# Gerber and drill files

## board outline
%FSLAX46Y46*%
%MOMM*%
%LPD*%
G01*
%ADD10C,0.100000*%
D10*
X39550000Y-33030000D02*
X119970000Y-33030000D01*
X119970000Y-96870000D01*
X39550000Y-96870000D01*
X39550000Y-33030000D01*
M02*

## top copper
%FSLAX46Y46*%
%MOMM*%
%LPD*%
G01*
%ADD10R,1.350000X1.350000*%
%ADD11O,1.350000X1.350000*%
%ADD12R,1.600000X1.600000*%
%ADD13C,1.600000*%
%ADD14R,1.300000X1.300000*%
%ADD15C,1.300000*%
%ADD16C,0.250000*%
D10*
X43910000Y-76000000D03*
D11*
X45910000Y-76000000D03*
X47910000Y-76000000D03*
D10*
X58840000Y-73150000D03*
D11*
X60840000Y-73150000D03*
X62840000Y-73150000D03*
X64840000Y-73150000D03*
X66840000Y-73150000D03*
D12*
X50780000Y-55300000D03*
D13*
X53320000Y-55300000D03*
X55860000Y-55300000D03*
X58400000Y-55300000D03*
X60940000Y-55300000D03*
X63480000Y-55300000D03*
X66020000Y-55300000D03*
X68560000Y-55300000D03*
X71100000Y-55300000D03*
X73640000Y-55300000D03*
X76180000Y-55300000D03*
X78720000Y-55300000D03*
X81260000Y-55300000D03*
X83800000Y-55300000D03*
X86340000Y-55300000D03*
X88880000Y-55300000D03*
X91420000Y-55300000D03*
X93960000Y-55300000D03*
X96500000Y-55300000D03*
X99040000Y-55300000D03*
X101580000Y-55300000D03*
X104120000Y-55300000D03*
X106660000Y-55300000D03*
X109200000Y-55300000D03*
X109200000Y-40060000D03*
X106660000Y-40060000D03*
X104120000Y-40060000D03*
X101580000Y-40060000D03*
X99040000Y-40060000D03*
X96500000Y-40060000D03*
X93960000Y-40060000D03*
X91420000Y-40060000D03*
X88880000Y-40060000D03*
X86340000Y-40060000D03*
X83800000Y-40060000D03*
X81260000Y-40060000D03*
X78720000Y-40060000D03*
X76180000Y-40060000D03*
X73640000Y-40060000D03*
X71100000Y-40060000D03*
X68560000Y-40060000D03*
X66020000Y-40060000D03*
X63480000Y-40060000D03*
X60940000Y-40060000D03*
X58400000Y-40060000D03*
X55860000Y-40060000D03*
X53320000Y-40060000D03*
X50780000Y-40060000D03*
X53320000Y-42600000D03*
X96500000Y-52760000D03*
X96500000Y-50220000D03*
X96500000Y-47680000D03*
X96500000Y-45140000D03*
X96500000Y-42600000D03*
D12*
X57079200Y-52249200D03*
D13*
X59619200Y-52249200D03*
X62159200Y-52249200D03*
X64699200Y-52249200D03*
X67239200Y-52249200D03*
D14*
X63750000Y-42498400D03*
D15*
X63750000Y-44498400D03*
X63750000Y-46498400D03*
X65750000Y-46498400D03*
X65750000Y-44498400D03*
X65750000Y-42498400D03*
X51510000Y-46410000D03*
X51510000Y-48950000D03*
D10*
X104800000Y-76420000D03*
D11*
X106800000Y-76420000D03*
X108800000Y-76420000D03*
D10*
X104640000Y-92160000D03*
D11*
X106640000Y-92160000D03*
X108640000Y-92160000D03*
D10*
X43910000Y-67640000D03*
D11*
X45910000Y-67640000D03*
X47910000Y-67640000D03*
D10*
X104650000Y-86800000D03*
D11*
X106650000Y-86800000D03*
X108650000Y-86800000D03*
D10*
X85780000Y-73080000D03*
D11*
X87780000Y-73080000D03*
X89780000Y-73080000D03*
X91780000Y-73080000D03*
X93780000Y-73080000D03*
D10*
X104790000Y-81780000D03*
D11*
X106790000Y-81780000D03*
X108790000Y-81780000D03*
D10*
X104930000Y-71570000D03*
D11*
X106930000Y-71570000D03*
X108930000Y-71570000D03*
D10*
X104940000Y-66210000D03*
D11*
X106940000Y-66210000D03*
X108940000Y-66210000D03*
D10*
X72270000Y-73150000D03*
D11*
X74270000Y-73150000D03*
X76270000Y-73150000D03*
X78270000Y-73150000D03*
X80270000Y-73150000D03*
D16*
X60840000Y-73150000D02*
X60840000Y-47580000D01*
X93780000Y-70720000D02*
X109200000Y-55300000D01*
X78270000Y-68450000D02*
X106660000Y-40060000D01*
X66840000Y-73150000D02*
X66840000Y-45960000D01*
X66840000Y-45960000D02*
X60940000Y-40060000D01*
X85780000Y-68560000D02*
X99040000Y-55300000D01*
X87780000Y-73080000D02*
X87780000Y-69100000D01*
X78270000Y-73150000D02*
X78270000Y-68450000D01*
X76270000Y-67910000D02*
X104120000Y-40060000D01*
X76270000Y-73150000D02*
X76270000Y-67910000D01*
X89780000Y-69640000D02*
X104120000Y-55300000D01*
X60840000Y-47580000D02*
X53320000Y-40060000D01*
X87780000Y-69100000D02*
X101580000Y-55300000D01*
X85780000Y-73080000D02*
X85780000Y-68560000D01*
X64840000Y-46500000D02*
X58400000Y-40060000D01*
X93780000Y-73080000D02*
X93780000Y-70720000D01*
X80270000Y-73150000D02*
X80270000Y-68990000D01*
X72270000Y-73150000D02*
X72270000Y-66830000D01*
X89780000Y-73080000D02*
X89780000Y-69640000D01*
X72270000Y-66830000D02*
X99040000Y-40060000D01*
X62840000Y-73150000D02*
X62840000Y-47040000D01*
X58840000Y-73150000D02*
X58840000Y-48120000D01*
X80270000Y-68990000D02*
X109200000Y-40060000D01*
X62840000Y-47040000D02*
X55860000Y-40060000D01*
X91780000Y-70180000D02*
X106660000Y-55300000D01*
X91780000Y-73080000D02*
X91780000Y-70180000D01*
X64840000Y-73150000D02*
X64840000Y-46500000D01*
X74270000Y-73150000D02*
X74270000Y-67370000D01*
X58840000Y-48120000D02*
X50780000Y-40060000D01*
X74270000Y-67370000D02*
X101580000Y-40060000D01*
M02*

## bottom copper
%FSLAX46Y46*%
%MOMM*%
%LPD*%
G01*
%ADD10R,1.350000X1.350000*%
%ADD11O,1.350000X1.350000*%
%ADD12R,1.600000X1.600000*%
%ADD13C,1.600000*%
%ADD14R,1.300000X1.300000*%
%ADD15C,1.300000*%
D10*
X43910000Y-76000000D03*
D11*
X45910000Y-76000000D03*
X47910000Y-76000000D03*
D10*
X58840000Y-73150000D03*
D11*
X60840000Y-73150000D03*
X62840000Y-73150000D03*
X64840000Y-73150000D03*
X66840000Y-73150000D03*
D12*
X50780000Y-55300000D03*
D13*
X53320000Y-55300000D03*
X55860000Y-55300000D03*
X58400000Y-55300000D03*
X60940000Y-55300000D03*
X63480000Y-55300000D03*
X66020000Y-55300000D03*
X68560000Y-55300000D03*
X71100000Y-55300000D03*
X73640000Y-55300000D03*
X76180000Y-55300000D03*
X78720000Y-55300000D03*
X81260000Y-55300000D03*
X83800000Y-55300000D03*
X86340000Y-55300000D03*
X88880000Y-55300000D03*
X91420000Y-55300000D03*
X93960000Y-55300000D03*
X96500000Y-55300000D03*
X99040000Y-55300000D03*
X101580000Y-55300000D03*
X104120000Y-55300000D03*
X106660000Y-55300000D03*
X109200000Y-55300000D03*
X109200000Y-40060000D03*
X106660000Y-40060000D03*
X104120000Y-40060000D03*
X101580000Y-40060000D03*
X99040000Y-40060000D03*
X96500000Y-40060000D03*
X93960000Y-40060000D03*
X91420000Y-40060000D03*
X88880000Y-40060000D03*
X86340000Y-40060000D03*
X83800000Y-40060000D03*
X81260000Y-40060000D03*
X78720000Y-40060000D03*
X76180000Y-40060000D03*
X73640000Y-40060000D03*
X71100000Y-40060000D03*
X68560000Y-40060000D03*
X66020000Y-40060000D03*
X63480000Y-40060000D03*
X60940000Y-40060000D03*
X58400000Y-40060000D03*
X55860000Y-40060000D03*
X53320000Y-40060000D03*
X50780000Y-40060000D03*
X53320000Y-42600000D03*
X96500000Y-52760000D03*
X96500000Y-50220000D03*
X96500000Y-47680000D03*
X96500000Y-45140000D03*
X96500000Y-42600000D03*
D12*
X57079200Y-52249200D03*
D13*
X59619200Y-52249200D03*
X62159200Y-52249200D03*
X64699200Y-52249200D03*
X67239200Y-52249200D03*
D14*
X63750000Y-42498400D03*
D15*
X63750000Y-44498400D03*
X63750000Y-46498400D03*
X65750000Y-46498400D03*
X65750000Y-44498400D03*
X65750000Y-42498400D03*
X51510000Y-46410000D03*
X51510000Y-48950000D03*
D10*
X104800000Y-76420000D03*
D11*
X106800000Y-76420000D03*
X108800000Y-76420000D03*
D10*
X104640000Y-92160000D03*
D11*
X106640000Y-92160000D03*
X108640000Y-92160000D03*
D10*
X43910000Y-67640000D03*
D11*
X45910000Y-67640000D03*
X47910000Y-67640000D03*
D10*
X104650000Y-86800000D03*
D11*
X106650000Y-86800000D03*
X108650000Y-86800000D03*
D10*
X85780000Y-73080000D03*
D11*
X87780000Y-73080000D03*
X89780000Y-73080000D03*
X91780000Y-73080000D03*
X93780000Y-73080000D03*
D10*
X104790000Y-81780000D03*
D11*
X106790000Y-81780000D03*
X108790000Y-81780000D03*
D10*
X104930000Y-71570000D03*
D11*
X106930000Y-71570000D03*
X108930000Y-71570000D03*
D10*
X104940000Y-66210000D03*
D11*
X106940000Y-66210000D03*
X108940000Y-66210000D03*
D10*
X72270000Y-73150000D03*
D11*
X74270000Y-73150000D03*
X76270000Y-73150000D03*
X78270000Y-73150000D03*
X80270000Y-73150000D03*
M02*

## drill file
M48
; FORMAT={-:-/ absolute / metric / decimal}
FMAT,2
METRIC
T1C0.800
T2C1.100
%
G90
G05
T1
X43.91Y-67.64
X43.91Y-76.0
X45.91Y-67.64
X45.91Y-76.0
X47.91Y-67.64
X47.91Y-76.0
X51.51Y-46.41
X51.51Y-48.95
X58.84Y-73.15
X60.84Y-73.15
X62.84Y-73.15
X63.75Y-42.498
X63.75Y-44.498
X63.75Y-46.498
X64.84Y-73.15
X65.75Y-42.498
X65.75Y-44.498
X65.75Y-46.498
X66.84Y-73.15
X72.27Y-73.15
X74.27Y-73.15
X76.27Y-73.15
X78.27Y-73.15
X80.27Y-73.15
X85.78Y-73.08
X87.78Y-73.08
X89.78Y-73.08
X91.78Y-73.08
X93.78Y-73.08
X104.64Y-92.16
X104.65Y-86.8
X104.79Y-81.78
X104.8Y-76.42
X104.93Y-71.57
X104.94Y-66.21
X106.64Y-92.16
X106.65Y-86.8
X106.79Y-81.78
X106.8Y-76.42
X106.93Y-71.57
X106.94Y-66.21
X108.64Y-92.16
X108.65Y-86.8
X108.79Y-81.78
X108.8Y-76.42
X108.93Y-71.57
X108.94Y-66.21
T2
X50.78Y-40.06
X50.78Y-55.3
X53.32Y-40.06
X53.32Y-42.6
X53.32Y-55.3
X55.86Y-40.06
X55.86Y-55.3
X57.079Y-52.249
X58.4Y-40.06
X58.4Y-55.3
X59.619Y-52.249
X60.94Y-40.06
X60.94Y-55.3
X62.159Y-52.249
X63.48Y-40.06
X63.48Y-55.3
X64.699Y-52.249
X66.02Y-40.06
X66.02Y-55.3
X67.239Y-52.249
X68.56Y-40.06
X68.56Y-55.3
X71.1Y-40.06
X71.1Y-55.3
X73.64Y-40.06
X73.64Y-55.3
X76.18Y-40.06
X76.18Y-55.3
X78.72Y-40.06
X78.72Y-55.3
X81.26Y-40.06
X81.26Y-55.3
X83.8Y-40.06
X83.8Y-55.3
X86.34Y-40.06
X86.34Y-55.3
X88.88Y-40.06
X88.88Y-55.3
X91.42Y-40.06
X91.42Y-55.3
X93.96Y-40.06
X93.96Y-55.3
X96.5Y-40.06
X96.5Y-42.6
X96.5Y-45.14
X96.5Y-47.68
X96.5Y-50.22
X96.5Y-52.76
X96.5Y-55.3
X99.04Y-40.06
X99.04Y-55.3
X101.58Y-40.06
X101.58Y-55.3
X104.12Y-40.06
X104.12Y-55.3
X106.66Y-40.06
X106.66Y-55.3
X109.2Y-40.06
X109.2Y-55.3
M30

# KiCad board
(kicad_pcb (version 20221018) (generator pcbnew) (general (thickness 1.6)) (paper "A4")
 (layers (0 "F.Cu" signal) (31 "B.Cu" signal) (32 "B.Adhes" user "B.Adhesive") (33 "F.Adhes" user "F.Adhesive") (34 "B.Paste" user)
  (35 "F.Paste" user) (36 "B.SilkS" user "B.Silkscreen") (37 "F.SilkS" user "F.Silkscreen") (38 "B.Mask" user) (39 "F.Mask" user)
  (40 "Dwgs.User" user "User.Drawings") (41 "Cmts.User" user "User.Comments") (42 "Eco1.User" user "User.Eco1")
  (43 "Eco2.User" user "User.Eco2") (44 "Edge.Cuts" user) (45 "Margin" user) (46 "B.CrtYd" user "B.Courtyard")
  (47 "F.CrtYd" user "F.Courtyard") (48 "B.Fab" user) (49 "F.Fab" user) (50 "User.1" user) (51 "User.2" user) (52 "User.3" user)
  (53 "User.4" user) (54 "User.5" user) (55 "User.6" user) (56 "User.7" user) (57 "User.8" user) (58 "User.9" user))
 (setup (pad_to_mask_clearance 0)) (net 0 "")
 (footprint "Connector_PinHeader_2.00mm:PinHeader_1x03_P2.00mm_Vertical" (layer "F.Cu") (at 43.91 76 90)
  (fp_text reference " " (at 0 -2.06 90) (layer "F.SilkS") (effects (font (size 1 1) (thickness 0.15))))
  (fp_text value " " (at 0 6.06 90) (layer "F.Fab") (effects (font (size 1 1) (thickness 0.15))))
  (pad "1" thru_hole rect (at 0 0 90) (size 1.35 1.35) (drill 0.8) (layers "*.Cu" "*.Mask"))
  (pad "2" thru_hole oval (at 0 2 90) (size 1.35 1.35) (drill 0.8) (layers "*.Cu" "*.Mask"))
  (pad "3" thru_hole oval (at 0 4 90) (size 1.35 1.35) (drill 0.8) (layers "*.Cu" "*.Mask")))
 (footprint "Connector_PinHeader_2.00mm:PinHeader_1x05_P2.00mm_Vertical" (layer "F.Cu") (at 58.84 73.15 90)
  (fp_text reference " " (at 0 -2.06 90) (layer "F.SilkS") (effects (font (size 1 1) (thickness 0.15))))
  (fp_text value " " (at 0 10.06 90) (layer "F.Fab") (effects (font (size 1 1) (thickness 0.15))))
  (pad "1" thru_hole rect (at 0 0 90) (size 1.35 1.35) (drill 0.8) (layers "*.Cu" "*.Mask"))
  (pad "2" thru_hole oval (at 0 2 90) (size 1.35 1.35) (drill 0.8) (layers "*.Cu" "*.Mask"))
  (pad "3" thru_hole oval (at 0 4 90) (size 1.35 1.35) (drill 0.8) (layers "*.Cu" "*.Mask"))
  (pad "4" thru_hole oval (at 0 6 90) (size 1.35 1.35) (drill 0.8) (layers "*.Cu" "*.Mask"))
  (pad "5" thru_hole oval (at 0 8 90) (size 1.35 1.35) (drill 0.8) (layers "*.Cu" "*.Mask")))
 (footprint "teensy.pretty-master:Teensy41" (layer "F.Cu") (at 79.99 47.68)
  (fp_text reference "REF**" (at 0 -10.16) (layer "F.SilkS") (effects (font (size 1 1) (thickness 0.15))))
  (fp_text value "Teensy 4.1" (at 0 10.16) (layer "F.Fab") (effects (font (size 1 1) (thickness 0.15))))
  (pad "1" thru_hole rect (at -29.21 7.62) (size 1.6 1.6) (drill 1.1) (layers "*.Cu" "*.Mask"))
  (pad "2" thru_hole circle (at -26.67 7.62) (size 1.6 1.6) (drill 1.1) (layers "*.Cu" "*.Mask"))
  (pad "3" thru_hole circle (at -24.13 7.62) (size 1.6 1.6) (drill 1.1) (layers "*.Cu" "*.Mask"))
  (pad "4" thru_hole circle (at -21.59 7.62) (size 1.6 1.6) (drill 1.1) (layers "*.Cu" "*.Mask"))
  (pad "5" thru_hole circle (at -19.05 7.62) (size 1.6 1.6) (drill 1.1) (layers "*.Cu" "*.Mask"))
  (pad "6" thru_hole circle (at -16.51 7.62) (size 1.6 1.6) (drill 1.1) (layers "*.Cu" "*.Mask"))
  (pad "7" thru_hole circle (at -13.97 7.62) (size 1.6 1.6) (drill 1.1) (layers "*.Cu" "*.Mask"))
  (pad "8" thru_hole circle (at -11.43 7.62) (size 1.6 1.6) (drill 1.1) (layers "*.Cu" "*.Mask"))
  (pad "9" thru_hole circle (at -8.89 7.62) (size 1.6 1.6) (drill 1.1) (layers "*.Cu" "*.Mask"))
  (pad "10" thru_hole circle (at -6.35 7.62) (size 1.6 1.6) (drill 1.1) (layers "*.Cu" "*.Mask"))
  (pad "11" thru_hole circle (at -3.81 7.62) (size 1.6 1.6) (drill 1.1) (layers "*.Cu" "*.Mask"))
  (pad "12" thru_hole circle (at -1.27 7.62) (size 1.6 1.6) (drill 1.1) (layers "*.Cu" "*.Mask"))
  (pad "13" thru_hole circle (at 1.27 7.62) (size 1.6 1.6) (drill 1.1) (layers "*.Cu" "*.Mask"))
  (pad "14" thru_hole circle (at 3.81 7.62) (size 1.6 1.6) (drill 1.1) (layers "*.Cu" "*.Mask"))
  (pad "15" thru_hole circle (at 6.35 7.62) (size 1.6 1.6) (drill 1.1) (layers "*.Cu" "*.Mask"))
  (pad "16" thru_hole circle (at 8.89 7.62) (size 1.6 1.6) (drill 1.1) (layers "*.Cu" "*.Mask"))
  (pad "17" thru_hole circle (at 11.43 7.62) (size 1.6 1.6) (drill 1.1) (layers "*.Cu" "*.Mask"))
  (pad "18" thru_hole circle (at 13.97 7.62) (size 1.6 1.6) (drill 1.1) (layers "*.Cu" "*.Mask"))
  (pad "19" thru_hole circle (at 16.51 7.62) (size 1.6 1.6) (drill 1.1) (layers "*.Cu" "*.Mask"))
  (pad "20" thru_hole circle (at 19.05 7.62) (size 1.6 1.6) (drill 1.1) (layers "*.Cu" "*.Mask"))
  (pad "21" thru_hole circle (at 21.59 7.62) (size 1.6 1.6) (drill 1.1) (layers "*.Cu" "*.Mask"))
  (pad "22" thru_hole circle (at 24.13 7.62) (size 1.6 1.6) (drill 1.1) (layers "*.Cu" "*.Mask"))
  (pad "23" thru_hole circle (at 26.67 7.62) (size 1.6 1.6) (drill 1.1) (layers "*.Cu" "*.Mask"))
  (pad "24" thru_hole circle (at 29.21 7.62) (size 1.6 1.6) (drill 1.1) (layers "*.Cu" "*.Mask"))
  (pad "25" thru_hole circle (at 29.21 -7.62) (size 1.6 1.6) (drill 1.1) (layers "*.Cu" "*.Mask"))
  (pad "26" thru_hole circle (at 26.67 -7.62) (size 1.6 1.6) (drill 1.1) (layers "*.Cu" "*.Mask"))
  (pad "27" thru_hole circle (at 24.13 -7.62) (size 1.6 1.6) (drill 1.1) (layers "*.Cu" "*.Mask"))
  (pad "28" thru_hole circle (at 21.59 -7.62) (size 1.6 1.6) (drill 1.1) (layers "*.Cu" "*.Mask"))
  (pad "29" thru_hole circle (at 19.05 -7.62) (size 1.6 1.6) (drill 1.1) (layers "*.Cu" "*.Mask"))
  (pad "30" thru_hole circle (at 16.51 -7.62) (size 1.6 1.6) (drill 1.1) (layers "*.Cu" "*.Mask"))
  (pad "31" thru_hole circle (at 13.97 -7.62) (size 1.6 1.6) (drill 1.1) (layers "*.Cu" "*.Mask"))
  (pad "32" thru_hole circle (at 11.43 -7.62) (size 1.6 1.6) (drill 1.1) (layers "*.Cu" "*.Mask"))
  (pad "33" thru_hole circle (at 8.89 -7.62) (size 1.6 1.6) (drill 1.1) (layers "*.Cu" "*.Mask"))
  (pad "34" thru_hole circle (at 6.35 -7.62) (size 1.6 1.6) (drill 1.1) (layers "*.Cu" "*.Mask"))
  (pad "35" thru_hole circle (at 3.81 -7.62) (size 1.6 1.6) (drill 1.1) (layers "*.Cu" "*.Mask"))
  (pad "36" thru_hole circle (at 1.27 -7.62) (size 1.6 1.6) (drill 1.1) (layers "*.Cu" "*.Mask"))
  (pad "37" thru_hole circle (at -1.27 -7.62) (size 1.6 1.6) (drill 1.1) (layers "*.Cu" "*.Mask"))
  (pad "38" thru_hole circle (at -3.81 -7.62) (size 1.6 1.6) (drill 1.1) (layers "*.Cu" "*.Mask"))
  (pad "39" thru_hole circle (at -6.35 -7.62) (size 1.6 1.6) (drill 1.1) (layers "*.Cu" "*.Mask"))
  (pad "40" thru_hole circle (at -8.89 -7.62) (size 1.6 1.6) (drill 1.1) (layers "*.Cu" "*.Mask"))
  (pad "41" thru_hole circle (at -11.43 -7.62) (size 1.6 1.6) (drill 1.1) (layers "*.Cu" "*.Mask"))
  (pad "42" thru_hole circle (at -13.97 -7.62) (size 1.6 1.6) (drill 1.1) (layers "*.Cu" "*.Mask"))
  (pad "43" thru_hole circle (at -16.51 -7.62) (size 1.6 1.6) (drill 1.1) (layers "*.Cu" "*.Mask"))
  (pad "44" thru_hole circle (at -19.05 -7.62) (size 1.6 1.6) (drill 1.1) (layers "*.Cu" "*.Mask"))
  (pad "45" thru_hole circle (at -21.59 -7.62) (size 1.6 1.6) (drill 1.1) (layers "*.Cu" "*.Mask"))
  (pad "46" thru_hole circle (at -24.13 -7.62) (size 1.6 1.6) (drill 1.1) (layers "*.Cu" "*.Mask"))
  (pad "47" thru_hole circle (at -26.67 -7.62) (size 1.6 1.6) (drill 1.1) (layers "*.Cu" "*.Mask"))
  (pad "48" thru_hole circle (at -29.21 -7.62) (size 1.6 1.6) (drill 1.1) (layers "*.Cu" "*.Mask"))
  (pad "49" thru_hole circle (at -26.67 -5.08) (size 1.6 1.6) (drill 1.1) (layers "*.Cu" "*.Mask"))
  (pad "50" thru_hole circle (at 16.51 5.08) (size 1.6 1.6) (drill 1.1) (layers "*.Cu" "*.Mask"))
  (pad "51" thru_hole circle (at 16.51 2.54) (size 1.6 1.6) (drill 1.1) (layers "*.Cu" "*.Mask"))
  (pad "52" thru_hole circle (at 16.51 0) (size 1.6 1.6) (drill 1.1) (layers "*.Cu" "*.Mask"))
  (pad "53" thru_hole circle (at 16.51 -2.54) (size 1.6 1.6) (drill 1.1) (layers "*.Cu" "*.Mask"))
  (pad "54" thru_hole circle (at 16.51 -5.08) (size 1.6 1.6) (drill 1.1) (layers "*.Cu" "*.Mask"))
  (pad "55" thru_hole rect (at -22.9108 4.5692) (size 1.6 1.6) (drill 1.1) (layers "*.Cu" "*.Mask"))
  (pad "56" thru_hole circle (at -20.3708 4.5692) (size 1.6 1.6) (drill 1.1) (layers "*.Cu" "*.Mask"))
  (pad "57" thru_hole circle (at -17.8308 4.5692) (size 1.6 1.6) (drill 1.1) (layers "*.Cu" "*.Mask"))
  (pad "58" thru_hole circle (at -15.2908 4.5692) (size 1.6 1.6) (drill 1.1) (layers "*.Cu" "*.Mask"))
  (pad "59" thru_hole circle (at -12.7508 4.5692) (size 1.6 1.6) (drill 1.1) (layers "*.Cu" "*.Mask"))
  (pad "60" thru_hole rect (at -16.24 -5.1816) (size 1.3 1.3) (drill 0.8) (layers "*.Cu" "*.Mask"))
  (pad "61" thru_hole circle (at -16.24 -3.1816) (size 1.3 1.3) (drill 0.8) (layers "*.Cu" "*.Mask"))
  (pad "62" thru_hole circle (at -16.24 -1.1816) (size 1.3 1.3) (drill 0.8) (layers "*.Cu" "*.Mask"))
  (pad "63" thru_hole circle (at -14.24 -1.1816) (size 1.3 1.3) (drill 0.8) (layers "*.Cu" "*.Mask"))
  (pad "64" thru_hole circle (at -14.24 -3.1816) (size 1.3 1.3) (drill 0.8) (layers "*.Cu" "*.Mask"))
  (pad "65" thru_hole circle (at -14.24 -5.1816) (size 1.3 1.3) (drill 0.8) (layers "*.Cu" "*.Mask"))
  (pad "66" thru_hole circle (at -28.48 -1.27) (size 1.3 1.3) (drill 0.8) (layers "*.Cu" "*.Mask"))
  (pad "67" thru_hole circle (at -28.48 1.27) (size 1.3 1.3) (drill 0.8) (layers "*.Cu" "*.Mask")))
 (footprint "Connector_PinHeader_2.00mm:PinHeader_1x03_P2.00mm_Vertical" (layer "F.Cu") (at 104.8 76.42 90)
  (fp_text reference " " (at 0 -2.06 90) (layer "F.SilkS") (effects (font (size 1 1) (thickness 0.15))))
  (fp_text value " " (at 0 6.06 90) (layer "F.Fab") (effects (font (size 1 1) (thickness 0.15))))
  (pad "1" thru_hole rect (at 0 0 90) (size 1.35 1.35) (drill 0.8) (layers "*.Cu" "*.Mask"))
  (pad "2" thru_hole oval (at 0 2 90) (size 1.35 1.35) (drill 0.8) (layers "*.Cu" "*.Mask"))
  (pad "3" thru_hole oval (at 0 4 90) (size 1.35 1.35) (drill 0.8) (layers "*.Cu" "*.Mask")))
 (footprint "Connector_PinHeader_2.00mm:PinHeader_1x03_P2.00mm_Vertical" (layer "F.Cu") (at 104.64 92.16 90)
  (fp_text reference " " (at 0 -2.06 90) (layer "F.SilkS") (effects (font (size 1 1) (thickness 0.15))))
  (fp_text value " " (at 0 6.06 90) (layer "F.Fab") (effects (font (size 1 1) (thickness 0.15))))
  (pad "1" thru_hole rect (at 0 0 90) (size 1.35 1.35) (drill 0.8) (layers "*.Cu" "*.Mask"))
  (pad "2" thru_hole oval (at 0 2 90) (size 1.35 1.35) (drill 0.8) (layers "*.Cu" "*.Mask"))
  (pad "3" thru_hole oval (at 0 4 90) (size 1.35 1.35) (drill 0.8) (layers "*.Cu" "*.Mask")))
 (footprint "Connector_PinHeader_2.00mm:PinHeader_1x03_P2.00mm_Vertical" (layer "F.Cu") (at 43.91 67.64 90)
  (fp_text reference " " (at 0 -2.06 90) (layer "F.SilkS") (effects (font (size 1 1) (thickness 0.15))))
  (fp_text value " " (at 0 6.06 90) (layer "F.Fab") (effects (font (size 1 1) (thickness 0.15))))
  (pad "1" thru_hole rect (at 0 0 90) (size 1.35 1.35) (drill 0.8) (layers "*.Cu" "*.Mask"))
  (pad "2" thru_hole oval (at 0 2 90) (size 1.35 1.35) (drill 0.8) (layers "*.Cu" "*.Mask"))
  (pad "3" thru_hole oval (at 0 4 90) (size 1.35 1.35) (drill 0.8) (layers "*.Cu" "*.Mask")))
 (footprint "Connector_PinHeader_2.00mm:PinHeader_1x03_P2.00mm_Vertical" (layer "F.Cu") (at 104.65 86.8 90)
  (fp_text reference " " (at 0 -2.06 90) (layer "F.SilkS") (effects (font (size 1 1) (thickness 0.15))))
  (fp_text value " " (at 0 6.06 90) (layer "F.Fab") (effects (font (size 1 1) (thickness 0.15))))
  (pad "1" thru_hole rect (at 0 0 90) (size 1.35 1.35) (drill 0.8) (layers "*.Cu" "*.Mask"))
  (pad "2" thru_hole oval (at 0 2 90) (size 1.35 1.35) (drill 0.8) (layers "*.Cu" "*.Mask"))
  (pad "3" thru_hole oval (at 0 4 90) (size 1.35 1.35) (drill 0.8) (layers "*.Cu" "*.Mask")))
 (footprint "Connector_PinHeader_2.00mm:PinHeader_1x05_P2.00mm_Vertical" (layer "F.Cu") (at 85.78 73.08 90)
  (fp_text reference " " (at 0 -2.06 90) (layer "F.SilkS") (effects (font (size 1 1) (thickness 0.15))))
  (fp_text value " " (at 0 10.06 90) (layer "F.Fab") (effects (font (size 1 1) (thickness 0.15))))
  (pad "1" thru_hole rect (at 0 0 90) (size 1.35 1.35) (drill 0.8) (layers "*.Cu" "*.Mask"))
  (pad "2" thru_hole oval (at 0 2 90) (size 1.35 1.35) (drill 0.8) (layers "*.Cu" "*.Mask"))
  (pad "3" thru_hole oval (at 0 4 90) (size 1.35 1.35) (drill 0.8) (layers "*.Cu" "*.Mask"))
  (pad "4" thru_hole oval (at 0 6 90) (size 1.35 1.35) (drill 0.8) (layers "*.Cu" "*.Mask"))
  (pad "5" thru_hole oval (at 0 8 90) (size 1.35 1.35) (drill 0.8) (layers "*.Cu" "*.Mask")))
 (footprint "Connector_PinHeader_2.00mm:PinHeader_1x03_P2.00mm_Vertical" (layer "F.Cu") (at 104.79 81.78 90)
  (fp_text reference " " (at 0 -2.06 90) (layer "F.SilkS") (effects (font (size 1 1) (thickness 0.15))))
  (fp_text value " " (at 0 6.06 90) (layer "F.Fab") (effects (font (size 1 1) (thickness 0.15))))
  (pad "1" thru_hole rect (at 0 0 90) (size 1.35 1.35) (drill 0.8) (layers "*.Cu" "*.Mask"))
  (pad "2" thru_hole oval (at 0 2 90) (size 1.35 1.35) (drill 0.8) (layers "*.Cu" "*.Mask"))
  (pad "3" thru_hole oval (at 0 4 90) (size 1.35 1.35) (drill 0.8) (layers "*.Cu" "*.Mask")))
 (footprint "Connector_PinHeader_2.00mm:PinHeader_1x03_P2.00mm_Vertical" (layer "F.Cu") (at 104.93 71.57 90)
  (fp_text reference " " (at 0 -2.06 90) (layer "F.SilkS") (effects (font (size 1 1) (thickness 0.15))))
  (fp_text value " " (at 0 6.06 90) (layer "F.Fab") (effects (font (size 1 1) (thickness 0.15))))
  (pad "1" thru_hole rect (at 0 0 90) (size 1.35 1.35) (drill 0.8) (layers "*.Cu" "*.Mask"))
  (pad "2" thru_hole oval (at 0 2 90) (size 1.35 1.35) (drill 0.8) (layers "*.Cu" "*.Mask"))
  (pad "3" thru_hole oval (at 0 4 90) (size 1.35 1.35) (drill 0.8) (layers "*.Cu" "*.Mask")))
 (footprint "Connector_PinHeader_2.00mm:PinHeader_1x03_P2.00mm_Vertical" (layer "F.Cu") (at 104.94 66.21 90)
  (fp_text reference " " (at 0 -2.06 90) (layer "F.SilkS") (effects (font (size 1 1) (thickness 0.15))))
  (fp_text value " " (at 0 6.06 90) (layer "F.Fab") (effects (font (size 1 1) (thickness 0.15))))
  (pad "1" thru_hole rect (at 0 0 90) (size 1.35 1.35) (drill 0.8) (layers "*.Cu" "*.Mask"))
  (pad "2" thru_hole oval (at 0 2 90) (size 1.35 1.35) (drill 0.8) (layers "*.Cu" "*.Mask"))
  (pad "3" thru_hole oval (at 0 4 90) (size 1.35 1.35) (drill 0.8) (layers "*.Cu" "*.Mask")))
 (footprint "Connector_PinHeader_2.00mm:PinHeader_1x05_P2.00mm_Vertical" (layer "F.Cu") (at 72.27 73.15 90)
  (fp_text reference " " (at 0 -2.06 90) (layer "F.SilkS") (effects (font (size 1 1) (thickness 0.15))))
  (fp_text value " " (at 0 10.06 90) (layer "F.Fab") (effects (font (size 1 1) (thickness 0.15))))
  (pad "1" thru_hole rect (at 0 0 90) (size 1.35 1.35) (drill 0.8) (layers "*.Cu" "*.Mask"))
  (pad "2" thru_hole oval (at 0 2 90) (size 1.35 1.35) (drill 0.8) (layers "*.Cu" "*.Mask"))
  (pad "3" thru_hole oval (at 0 4 90) (size 1.35 1.35) (drill 0.8) (layers "*.Cu" "*.Mask"))
  (pad "4" thru_hole oval (at 0 6 90) (size 1.35 1.35) (drill 0.8) (layers "*.Cu" "*.Mask"))
  (pad "5" thru_hole oval (at 0 8 90) (size 1.35 1.35) (drill 0.8) (layers "*.Cu" "*.Mask")))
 (gr_rect (start 39.55 33.03) (end 119.97 96.87) (stroke (width 0.1) (type default)) (fill none) (layer "Edge.Cuts"))
 (segment (start 60.84 73.15) (end 60.84 47.58) (width 0.25) (layer "F.Cu") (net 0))
 (segment (start 93.78 70.72) (end 109.2 55.3) (width 0.25) (layer "F.Cu") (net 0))
 (segment (start 78.27 68.45) (end 106.66 40.06) (width 0.25) (layer "F.Cu") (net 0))
 (segment (start 66.84 73.15) (end 66.84 45.96) (width 0.25) (layer "F.Cu") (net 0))
 (segment (start 66.84 45.96) (end 60.94 40.06) (width 0.25) (layer "F.Cu") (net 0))
 (segment (start 85.78 68.56) (end 99.04 55.3) (width 0.25) (layer "F.Cu") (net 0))
 (segment (start 87.78 73.08) (end 87.78 69.1) (width 0.25) (layer "F.Cu") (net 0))
 (segment (start 78.27 73.15) (end 78.27 68.45) (width 0.25) (layer "F.Cu") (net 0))
 (segment (start 76.27 67.91) (end 104.12 40.06) (width 0.25) (layer "F.Cu") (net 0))
 (segment (start 76.27 73.15) (end 76.27 67.91) (width 0.25) (layer "F.Cu") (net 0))
 (segment (start 89.78 69.64) (end 104.12 55.3) (width 0.25) (layer "F.Cu") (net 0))
 (segment (start 60.84 47.58) (end 53.32 40.06) (width 0.25) (layer "F.Cu") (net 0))
 (segment (start 87.78 69.1) (end 101.58 55.3) (width 0.25) (layer "F.Cu") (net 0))
 (segment (start 85.78 73.08) (end 85.78 68.56) (width 0.25) (layer "F.Cu") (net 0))
 (segment (start 64.84 46.5) (end 58.4 40.06) (width 0.25) (layer "F.Cu") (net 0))
 (segment (start 93.78 73.08) (end 93.78 70.72) (width 0.25) (layer "F.Cu") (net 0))
 (segment (start 80.27 73.15) (end 80.27 68.99) (width 0.25) (layer "F.Cu") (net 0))
 (segment (start 72.27 73.15) (end 72.27 66.83) (width 0.25) (layer "F.Cu") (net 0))
 (segment (start 89.78 73.08) (end 89.78 69.64) (width 0.25) (layer "F.Cu") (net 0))
 (segment (start 72.27 66.83) (end 99.04 40.06) (width 0.25) (layer "F.Cu") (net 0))
 (segment (start 62.84 73.15) (end 62.84 47.04) (width 0.25) (layer "F.Cu") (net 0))
 (segment (start 58.84 73.15) (end 58.84 48.12) (width 0.25) (layer "F.Cu") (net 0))
 (segment (start 80.27 68.99) (end 109.2 40.06) (width 0.25) (layer "F.Cu") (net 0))
 (segment (start 62.84 47.04) (end 55.86 40.06) (width 0.25) (layer "F.Cu") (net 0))
 (segment (start 91.78 70.18) (end 106.66 55.3) (width 0.25) (layer "F.Cu") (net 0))
 (segment (start 91.78 73.08) (end 91.78 70.18) (width 0.25) (layer "F.Cu") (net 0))
 (segment (start 64.84 73.15) (end 64.84 46.5) (width 0.25) (layer "F.Cu") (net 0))
 (segment (start 74.27 73.15) (end 74.27 67.37) (width 0.25) (layer "F.Cu") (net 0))
 (segment (start 58.84 48.12) (end 50.78 40.06) (width 0.25) (layer "F.Cu") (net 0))
 (segment (start 74.27 67.37) (end 101.58 40.06) (width 0.25) (layer "F.Cu") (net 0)))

